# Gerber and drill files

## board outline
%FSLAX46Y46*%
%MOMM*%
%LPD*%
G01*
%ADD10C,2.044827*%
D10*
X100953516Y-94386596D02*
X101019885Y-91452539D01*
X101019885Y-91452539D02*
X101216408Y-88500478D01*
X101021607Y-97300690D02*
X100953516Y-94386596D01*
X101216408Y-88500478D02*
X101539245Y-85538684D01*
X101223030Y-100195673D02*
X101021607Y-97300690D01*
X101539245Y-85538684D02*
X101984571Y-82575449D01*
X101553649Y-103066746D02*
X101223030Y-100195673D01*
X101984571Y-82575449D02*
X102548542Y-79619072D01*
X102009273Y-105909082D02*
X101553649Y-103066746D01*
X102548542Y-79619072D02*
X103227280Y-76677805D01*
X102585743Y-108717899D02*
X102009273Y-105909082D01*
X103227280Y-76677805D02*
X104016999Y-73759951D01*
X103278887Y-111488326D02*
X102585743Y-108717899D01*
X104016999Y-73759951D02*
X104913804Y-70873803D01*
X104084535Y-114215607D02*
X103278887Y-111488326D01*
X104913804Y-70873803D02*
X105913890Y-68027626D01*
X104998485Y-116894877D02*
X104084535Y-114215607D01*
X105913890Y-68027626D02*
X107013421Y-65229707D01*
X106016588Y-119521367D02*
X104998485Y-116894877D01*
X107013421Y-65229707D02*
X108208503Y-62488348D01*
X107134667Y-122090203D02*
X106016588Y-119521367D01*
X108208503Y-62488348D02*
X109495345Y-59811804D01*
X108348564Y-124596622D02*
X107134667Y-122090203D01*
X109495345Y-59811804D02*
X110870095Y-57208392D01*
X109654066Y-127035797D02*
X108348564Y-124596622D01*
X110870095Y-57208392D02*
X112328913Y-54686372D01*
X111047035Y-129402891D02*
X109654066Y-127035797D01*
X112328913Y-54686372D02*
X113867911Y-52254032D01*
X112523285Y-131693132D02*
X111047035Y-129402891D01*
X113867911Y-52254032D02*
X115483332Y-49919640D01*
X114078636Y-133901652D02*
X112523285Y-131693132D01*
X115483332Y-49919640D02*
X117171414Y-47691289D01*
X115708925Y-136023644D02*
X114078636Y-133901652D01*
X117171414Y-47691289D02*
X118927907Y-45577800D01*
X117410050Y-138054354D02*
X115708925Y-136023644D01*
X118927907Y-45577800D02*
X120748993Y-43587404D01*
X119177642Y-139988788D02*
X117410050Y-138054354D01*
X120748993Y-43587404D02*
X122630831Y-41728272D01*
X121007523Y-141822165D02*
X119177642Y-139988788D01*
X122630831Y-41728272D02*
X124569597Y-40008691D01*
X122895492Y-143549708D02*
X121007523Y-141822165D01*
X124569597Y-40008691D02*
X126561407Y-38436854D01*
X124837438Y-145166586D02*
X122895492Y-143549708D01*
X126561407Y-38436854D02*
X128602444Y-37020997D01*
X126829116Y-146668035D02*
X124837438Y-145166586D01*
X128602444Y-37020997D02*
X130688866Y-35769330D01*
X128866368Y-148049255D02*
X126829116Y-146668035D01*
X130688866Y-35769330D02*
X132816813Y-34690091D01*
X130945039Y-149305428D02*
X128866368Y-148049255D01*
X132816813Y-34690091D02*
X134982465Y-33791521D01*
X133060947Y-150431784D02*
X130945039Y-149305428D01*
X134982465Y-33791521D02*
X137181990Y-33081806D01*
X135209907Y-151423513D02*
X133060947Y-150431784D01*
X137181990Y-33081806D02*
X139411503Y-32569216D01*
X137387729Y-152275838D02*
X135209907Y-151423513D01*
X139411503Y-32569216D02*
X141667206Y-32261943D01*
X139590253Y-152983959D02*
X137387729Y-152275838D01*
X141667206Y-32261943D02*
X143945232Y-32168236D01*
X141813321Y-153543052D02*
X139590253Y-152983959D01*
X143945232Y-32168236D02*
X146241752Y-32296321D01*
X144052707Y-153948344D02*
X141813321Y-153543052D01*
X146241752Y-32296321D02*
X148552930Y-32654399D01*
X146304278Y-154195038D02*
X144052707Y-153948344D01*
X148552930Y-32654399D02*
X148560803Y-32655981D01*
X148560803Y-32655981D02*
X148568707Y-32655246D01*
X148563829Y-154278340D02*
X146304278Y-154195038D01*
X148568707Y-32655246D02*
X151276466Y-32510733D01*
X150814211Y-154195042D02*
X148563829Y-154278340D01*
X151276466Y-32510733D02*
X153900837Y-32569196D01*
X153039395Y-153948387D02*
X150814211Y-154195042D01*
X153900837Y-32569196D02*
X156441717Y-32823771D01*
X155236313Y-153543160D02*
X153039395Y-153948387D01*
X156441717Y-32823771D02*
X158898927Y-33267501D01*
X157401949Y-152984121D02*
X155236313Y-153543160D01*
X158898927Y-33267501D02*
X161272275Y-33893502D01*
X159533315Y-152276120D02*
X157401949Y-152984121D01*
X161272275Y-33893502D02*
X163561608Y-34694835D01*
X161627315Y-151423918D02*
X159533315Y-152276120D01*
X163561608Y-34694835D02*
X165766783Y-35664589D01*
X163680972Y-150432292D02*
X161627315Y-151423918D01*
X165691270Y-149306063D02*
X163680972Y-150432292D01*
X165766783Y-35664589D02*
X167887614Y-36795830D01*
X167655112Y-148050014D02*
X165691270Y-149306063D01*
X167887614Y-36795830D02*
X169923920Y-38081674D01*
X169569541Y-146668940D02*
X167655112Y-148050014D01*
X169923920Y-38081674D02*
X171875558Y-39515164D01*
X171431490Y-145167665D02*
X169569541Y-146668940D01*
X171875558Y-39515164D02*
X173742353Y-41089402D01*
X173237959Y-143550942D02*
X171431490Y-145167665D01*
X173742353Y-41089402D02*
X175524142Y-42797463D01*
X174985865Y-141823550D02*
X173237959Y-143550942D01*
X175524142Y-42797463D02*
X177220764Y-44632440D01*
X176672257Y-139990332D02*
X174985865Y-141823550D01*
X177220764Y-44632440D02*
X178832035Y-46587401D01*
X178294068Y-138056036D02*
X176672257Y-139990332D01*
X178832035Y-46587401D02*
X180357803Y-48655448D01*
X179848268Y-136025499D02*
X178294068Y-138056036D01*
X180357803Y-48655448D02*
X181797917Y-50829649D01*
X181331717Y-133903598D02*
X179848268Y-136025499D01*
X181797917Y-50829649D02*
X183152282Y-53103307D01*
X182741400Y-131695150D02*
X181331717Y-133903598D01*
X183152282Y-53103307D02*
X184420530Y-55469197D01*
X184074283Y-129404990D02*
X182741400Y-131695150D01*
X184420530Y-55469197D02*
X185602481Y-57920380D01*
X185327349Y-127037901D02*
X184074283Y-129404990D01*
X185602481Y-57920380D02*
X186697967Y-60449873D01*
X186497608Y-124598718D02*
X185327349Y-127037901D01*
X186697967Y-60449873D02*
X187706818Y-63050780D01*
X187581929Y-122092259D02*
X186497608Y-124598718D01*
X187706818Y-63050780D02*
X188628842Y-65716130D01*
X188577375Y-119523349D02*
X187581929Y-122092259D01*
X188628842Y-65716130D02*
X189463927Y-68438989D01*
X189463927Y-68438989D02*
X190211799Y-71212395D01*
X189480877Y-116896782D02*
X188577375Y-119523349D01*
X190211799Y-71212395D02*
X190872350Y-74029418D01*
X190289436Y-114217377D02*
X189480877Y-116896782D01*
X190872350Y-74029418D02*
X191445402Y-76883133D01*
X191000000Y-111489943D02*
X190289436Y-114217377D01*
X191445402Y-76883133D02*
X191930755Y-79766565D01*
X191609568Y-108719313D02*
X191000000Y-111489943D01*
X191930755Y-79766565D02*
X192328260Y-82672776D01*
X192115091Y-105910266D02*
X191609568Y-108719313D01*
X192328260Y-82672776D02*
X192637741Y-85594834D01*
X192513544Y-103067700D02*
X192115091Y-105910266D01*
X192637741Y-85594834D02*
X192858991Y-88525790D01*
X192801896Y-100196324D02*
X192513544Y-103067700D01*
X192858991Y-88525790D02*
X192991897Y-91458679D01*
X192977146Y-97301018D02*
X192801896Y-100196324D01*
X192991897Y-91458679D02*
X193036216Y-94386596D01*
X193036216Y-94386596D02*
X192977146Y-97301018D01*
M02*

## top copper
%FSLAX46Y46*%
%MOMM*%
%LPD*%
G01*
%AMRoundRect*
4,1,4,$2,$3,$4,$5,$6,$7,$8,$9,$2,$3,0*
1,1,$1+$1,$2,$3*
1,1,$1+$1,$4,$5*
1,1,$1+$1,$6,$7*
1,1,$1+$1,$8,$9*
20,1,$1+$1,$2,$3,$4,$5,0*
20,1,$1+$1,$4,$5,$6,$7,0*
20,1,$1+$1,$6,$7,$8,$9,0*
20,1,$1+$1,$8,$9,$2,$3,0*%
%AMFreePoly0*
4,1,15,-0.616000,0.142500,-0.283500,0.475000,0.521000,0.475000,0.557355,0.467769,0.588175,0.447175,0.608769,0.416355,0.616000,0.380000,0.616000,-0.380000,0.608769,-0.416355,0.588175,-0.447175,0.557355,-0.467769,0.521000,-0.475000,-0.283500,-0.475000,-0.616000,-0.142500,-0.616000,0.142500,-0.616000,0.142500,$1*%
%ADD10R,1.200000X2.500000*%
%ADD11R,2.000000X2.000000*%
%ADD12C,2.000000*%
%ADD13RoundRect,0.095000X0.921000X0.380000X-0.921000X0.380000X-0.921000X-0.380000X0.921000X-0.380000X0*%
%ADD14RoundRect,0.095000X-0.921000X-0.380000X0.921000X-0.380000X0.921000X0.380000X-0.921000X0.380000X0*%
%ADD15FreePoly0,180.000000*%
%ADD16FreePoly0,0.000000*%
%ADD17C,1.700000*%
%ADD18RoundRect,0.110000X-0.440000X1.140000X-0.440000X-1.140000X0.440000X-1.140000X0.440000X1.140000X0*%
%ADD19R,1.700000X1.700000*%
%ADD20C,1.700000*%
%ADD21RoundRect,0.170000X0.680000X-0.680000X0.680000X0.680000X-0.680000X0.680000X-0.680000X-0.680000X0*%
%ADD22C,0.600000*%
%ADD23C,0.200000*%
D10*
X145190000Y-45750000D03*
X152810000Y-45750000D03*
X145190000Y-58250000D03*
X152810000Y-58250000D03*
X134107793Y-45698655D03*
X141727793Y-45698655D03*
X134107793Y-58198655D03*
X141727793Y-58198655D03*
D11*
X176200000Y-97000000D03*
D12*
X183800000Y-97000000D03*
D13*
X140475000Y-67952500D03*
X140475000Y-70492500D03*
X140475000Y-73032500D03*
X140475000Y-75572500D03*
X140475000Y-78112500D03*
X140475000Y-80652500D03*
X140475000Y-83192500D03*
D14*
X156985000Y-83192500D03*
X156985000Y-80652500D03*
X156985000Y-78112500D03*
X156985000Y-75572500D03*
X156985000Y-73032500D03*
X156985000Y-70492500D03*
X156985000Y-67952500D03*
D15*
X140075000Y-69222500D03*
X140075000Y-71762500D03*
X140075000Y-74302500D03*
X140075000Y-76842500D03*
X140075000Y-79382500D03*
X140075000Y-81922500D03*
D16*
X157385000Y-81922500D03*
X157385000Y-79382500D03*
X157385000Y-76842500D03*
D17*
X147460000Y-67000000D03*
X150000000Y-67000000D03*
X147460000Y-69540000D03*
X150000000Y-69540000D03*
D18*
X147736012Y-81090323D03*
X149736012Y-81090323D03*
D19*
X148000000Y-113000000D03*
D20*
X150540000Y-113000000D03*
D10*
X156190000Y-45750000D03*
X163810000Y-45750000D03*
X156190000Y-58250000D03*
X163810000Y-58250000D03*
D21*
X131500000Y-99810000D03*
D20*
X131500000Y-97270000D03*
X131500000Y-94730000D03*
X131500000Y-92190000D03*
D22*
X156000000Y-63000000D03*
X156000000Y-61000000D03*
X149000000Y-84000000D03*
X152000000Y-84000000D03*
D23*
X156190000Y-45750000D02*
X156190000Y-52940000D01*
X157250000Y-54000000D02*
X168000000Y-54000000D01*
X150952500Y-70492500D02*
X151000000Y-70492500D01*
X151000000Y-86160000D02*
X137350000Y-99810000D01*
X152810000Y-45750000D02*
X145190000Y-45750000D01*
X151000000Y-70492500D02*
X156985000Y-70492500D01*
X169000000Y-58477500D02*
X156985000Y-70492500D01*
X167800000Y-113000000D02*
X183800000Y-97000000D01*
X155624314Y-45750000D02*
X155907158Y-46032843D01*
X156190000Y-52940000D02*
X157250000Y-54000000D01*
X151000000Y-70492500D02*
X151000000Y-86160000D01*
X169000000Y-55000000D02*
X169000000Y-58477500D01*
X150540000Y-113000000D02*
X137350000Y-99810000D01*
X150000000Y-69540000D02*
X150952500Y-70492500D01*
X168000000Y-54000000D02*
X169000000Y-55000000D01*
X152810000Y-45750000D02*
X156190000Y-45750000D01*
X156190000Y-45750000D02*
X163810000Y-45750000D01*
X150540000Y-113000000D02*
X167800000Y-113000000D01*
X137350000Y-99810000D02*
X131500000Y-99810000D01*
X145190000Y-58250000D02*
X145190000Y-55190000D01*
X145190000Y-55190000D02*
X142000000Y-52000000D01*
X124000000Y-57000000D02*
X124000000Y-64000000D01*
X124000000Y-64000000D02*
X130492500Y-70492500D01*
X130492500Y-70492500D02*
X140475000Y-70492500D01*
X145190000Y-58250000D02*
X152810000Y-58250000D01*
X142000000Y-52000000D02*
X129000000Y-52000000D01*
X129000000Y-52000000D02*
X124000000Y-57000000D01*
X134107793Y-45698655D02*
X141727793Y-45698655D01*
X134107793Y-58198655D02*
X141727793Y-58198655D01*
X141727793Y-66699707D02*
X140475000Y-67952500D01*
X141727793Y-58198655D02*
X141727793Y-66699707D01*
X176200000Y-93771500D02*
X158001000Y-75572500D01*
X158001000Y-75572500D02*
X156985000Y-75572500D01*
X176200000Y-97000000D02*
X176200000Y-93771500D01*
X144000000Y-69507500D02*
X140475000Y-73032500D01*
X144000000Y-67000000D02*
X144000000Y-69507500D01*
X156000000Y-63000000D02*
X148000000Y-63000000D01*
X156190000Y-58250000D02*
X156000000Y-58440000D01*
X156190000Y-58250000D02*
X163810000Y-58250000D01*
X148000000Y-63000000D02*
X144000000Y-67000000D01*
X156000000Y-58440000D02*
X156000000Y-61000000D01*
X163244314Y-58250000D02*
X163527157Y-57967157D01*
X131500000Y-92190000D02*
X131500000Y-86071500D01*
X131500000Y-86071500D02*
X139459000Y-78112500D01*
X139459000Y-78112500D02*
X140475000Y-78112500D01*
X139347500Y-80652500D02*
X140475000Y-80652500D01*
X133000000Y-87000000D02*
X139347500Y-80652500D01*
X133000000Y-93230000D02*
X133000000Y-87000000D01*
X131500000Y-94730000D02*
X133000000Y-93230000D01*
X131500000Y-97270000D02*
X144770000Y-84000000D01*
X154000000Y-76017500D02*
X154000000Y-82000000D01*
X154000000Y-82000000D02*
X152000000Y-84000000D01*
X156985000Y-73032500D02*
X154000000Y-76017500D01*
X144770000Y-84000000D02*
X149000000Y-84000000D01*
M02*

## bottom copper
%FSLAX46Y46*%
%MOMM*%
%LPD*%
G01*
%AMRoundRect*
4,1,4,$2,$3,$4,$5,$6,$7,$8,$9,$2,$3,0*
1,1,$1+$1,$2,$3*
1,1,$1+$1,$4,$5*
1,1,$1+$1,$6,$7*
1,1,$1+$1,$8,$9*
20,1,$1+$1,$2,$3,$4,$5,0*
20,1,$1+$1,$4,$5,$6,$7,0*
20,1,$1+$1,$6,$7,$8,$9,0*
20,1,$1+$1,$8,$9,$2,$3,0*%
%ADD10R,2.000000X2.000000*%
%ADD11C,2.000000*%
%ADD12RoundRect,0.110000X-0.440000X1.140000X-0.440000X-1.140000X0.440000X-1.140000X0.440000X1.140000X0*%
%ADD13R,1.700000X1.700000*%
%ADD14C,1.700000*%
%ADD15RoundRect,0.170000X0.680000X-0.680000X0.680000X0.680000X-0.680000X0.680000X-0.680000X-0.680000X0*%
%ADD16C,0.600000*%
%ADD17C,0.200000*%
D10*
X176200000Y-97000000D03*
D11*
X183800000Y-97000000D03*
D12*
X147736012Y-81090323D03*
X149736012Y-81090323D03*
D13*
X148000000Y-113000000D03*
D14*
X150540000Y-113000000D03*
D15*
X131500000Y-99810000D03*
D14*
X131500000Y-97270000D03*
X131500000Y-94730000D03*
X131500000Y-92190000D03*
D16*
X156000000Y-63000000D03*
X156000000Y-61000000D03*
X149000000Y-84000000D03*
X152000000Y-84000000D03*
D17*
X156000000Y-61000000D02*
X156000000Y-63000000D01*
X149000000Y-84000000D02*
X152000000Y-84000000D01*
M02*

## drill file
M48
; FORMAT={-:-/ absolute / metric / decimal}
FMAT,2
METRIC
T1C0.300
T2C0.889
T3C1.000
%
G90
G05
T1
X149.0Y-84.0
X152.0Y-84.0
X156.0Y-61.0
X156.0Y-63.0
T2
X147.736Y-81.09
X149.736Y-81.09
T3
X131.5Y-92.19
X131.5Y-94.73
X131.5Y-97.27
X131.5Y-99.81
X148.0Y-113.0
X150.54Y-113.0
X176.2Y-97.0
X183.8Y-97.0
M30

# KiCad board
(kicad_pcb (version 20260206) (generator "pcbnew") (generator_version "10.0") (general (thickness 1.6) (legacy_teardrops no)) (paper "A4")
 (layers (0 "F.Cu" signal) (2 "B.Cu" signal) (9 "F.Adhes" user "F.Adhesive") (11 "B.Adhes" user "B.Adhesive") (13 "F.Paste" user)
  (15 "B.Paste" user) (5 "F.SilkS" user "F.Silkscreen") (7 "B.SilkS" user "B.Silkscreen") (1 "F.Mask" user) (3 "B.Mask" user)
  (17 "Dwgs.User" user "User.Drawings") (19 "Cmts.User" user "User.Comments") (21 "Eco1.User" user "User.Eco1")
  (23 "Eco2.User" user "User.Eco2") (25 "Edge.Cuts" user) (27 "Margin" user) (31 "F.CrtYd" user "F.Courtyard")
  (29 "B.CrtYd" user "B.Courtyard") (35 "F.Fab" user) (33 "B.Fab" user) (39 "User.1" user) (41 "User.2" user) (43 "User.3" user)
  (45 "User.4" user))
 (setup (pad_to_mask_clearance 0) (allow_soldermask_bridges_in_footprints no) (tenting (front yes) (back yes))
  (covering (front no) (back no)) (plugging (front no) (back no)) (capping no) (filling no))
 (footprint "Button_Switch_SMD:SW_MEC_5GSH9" (layer "F.Cu") (at 149 52)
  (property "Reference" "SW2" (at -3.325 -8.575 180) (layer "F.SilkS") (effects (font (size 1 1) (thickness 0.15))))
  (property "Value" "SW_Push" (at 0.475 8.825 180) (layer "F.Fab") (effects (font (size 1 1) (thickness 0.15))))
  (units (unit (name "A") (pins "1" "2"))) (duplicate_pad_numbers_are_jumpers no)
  (pad "1" smd rect (at -3.81 -6.25 90) (size 2.5 1.2) (layers "F.Cu" "F.Mask" "F.Paste") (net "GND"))
  (pad "1" smd rect (at 3.81 -6.25 90) (size 2.5 1.2) (layers "F.Cu" "F.Mask" "B.SilkS" "F.Paste") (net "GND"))
  (pad "2" smd rect (at -3.81 6.25 90) (size 2.5 1.2) (layers "F.Cu" "F.Mask" "F.Paste") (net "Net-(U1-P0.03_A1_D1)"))
  (pad "2" smd rect (at 3.81 6.25 90) (size 2.5 1.2) (layers "F.Cu" "F.Mask" "F.Paste") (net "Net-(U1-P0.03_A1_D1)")))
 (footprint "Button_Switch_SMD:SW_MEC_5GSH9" (layer "F.Cu") (at 137.917793 51.948655)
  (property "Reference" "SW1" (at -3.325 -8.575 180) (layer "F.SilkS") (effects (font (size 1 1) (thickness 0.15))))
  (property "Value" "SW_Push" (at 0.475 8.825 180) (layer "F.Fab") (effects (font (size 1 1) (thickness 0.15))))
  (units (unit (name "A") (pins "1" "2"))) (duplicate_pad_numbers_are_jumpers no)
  (pad "1" smd rect (at -3.81 -6.25 90) (size 2.5 1.2) (layers "F.Cu" "F.Mask" "F.Paste") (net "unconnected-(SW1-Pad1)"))
  (pad "1" smd rect (at 3.81 -6.25 90) (size 2.5 1.2) (layers "F.Cu" "F.Mask" "B.SilkS" "F.Paste") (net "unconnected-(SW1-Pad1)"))
  (pad "2" smd rect (at -3.81 6.25 90) (size 2.5 1.2) (layers "F.Cu" "F.Mask" "F.Paste") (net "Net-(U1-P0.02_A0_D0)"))
  (pad "2" smd rect (at 3.81 6.25 90) (size 2.5 1.2) (layers "F.Cu" "F.Mask" "F.Paste") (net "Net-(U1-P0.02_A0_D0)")))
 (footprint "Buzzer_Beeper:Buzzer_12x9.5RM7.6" (layer "F.Cu") (at 176.2 97)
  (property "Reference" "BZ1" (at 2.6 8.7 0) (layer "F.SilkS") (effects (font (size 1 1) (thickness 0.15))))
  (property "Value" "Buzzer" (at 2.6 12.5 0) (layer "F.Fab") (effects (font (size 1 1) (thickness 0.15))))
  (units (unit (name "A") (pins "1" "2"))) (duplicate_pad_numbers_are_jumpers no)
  (pad "1" thru_hole rect (at 0 0) (size 2 2) (drill 1) (layers "*.Cu" "*.Mask") (remove_unused_layers no) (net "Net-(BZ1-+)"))
  (pad "2" thru_hole circle (at 7.6 0) (size 2 2) (drill 1) (layers "*.Cu" "*.Mask") (remove_unused_layers no) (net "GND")))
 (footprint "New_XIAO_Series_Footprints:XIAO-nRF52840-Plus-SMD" (layer "F.Cu") (at 148.73 75.5725 90)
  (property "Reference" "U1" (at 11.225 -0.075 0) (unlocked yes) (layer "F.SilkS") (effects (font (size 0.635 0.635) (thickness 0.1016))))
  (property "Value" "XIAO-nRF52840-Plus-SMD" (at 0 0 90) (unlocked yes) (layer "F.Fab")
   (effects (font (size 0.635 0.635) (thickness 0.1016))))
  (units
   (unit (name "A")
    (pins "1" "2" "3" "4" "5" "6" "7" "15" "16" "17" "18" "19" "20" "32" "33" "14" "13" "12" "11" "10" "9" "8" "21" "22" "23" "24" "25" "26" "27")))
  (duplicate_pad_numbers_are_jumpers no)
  (pad "1" smd roundrect (at 7.62 -8.255 180) (size 2.032 0.95) (layers "F.Cu" "F.Mask" "F.Paste") (roundrect_rratio 0.1)
   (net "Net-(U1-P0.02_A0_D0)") (thermal_bridge_angle 45))
  (pad "2" smd roundrect (at 5.08 -8.255 180) (size 2.032 0.95) (layers "F.Cu" "F.Mask" "F.Paste") (roundrect_rratio 0.1)
   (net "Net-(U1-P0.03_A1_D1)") (thermal_bridge_angle 45))
  (pad "3" smd roundrect (at 2.54 -8.255 180) (size 2.032 0.95) (layers "F.Cu" "F.Mask" "F.Paste") (roundrect_rratio 0.1)
   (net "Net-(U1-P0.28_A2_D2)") (thermal_bridge_angle 45))
  (pad "4" smd roundrect (at 0 -8.255 180) (size 2.032 0.95) (layers "F.Cu" "F.Mask" "F.Paste") (roundrect_rratio 0.1)
   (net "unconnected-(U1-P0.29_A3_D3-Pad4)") (thermal_bridge_angle 45))
  (pad "5" smd roundrect (at -2.54 -8.255 180) (size 2.032 0.95) (layers "F.Cu" "F.Mask" "F.Paste") (roundrect_rratio 0.1)
   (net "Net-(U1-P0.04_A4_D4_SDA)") (thermal_bridge_angle 45))
  (pad "6" smd roundrect (at -5.08 -8.255 180) (size 2.032 0.95) (layers "F.Cu" "F.Mask" "F.Paste") (roundrect_rratio 0.1)
   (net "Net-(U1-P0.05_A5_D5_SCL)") (thermal_bridge_angle 45))
  (pad "7" smd roundrect (at -7.62 -8.255 180) (size 2.032 0.95) (layers "F.Cu" "F.Mask" "F.Paste") (roundrect_rratio 0.1)
   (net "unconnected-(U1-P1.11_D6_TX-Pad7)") (thermal_bridge_angle 45))
  (pad "8" smd roundrect (at -7.62 8.255) (size 2.032 0.95) (layers "F.Cu" "F.Mask" "F.Paste") (roundrect_rratio 0.1)
   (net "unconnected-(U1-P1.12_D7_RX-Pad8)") (thermal_bridge_angle 45))
  (pad "9" smd roundrect (at -5.08 8.255) (size 2.032 0.95) (layers "F.Cu" "F.Mask" "F.Paste") (roundrect_rratio 0.1)
   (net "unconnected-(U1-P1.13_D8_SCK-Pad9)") (thermal_bridge_angle 45))
  (pad "10" smd roundrect (at -2.54 8.255) (size 2.032 0.95) (layers "F.Cu" "F.Mask" "F.Paste") (roundrect_rratio 0.1)
   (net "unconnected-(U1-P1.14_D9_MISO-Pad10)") (thermal_bridge_angle 45))
  (pad "11" smd roundrect (at 0 8.255) (size 2.032 0.95) (layers "F.Cu" "F.Mask" "F.Paste") (roundrect_rratio 0.1) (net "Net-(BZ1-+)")
   (thermal_bridge_angle 45))
  (pad "12" smd roundrect (at 2.54 8.255) (size 2.032 0.95) (layers "F.Cu" "F.Mask" "F.Paste") (roundrect_rratio 0.1) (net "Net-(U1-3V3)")
   (thermal_bridge_angle 45))
  (pad "13" smd roundrect (at 5.08 8.255) (size 2.032 0.95) (layers "F.Cu" "F.Mask" "F.Paste") (roundrect_rratio 0.1) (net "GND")
   (thermal_bridge_angle 45))
  (pad "14" smd roundrect (at 7.62 8.255) (size 2.032 0.95) (layers "F.Cu" "F.Mask" "F.Paste") (roundrect_rratio 0.1)
   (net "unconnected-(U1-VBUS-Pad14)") (thermal_bridge_angle 45))
  (pad "15" smd roundrect (at 6.35 -8.655 180) (size 1.232 0.95) (layers "F.Cu" "F.Mask" "F.Paste") (roundrect_rratio 0.1)
   (chamfer_ratio 0.35) (chamfer top_left bottom_left) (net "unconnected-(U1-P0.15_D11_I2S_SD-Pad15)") (thermal_bridge_angle 45))
  (pad "16" smd roundrect (at 3.81 -8.655 180) (size 1.232 0.95) (layers "F.Cu" "F.Mask" "F.Paste") (roundrect_rratio 0.1)
   (chamfer_ratio 0.35) (chamfer top_left bottom_left) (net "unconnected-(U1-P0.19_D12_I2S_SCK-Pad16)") (thermal_bridge_angle 45))
  (pad "17" smd roundrect (at 1.27 -8.655 180) (size 1.232 0.95) (layers "F.Cu" "F.Mask" "F.Paste") (roundrect_rratio 0.1)
   (chamfer_ratio 0.35) (chamfer top_left bottom_left) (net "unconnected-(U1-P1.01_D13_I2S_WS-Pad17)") (thermal_bridge_angle 45))
  (pad "18" smd roundrect (at -1.27 -8.655 180) (size 1.232 0.95) (layers "F.Cu" "F.Mask" "F.Paste") (roundrect_rratio 0.1)
   (chamfer_ratio 0.35) (chamfer top_left bottom_left) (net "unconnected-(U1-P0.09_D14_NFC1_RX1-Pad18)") (thermal_bridge_angle 45))
  (pad "19" smd roundrect (at -3.81 -8.655 180) (size 1.232 0.95) (layers "F.Cu" "F.Mask" "F.Paste") (roundrect_rratio 0.1)
   (chamfer_ratio 0.35) (chamfer top_left bottom_left) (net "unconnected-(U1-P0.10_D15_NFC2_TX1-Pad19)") (thermal_bridge_angle 45))
  (pad "20" smd roundrect (at -6.35 -8.655 180) (size 1.232 0.95) (layers "F.Cu" "F.Mask" "F.Paste") (roundrect_rratio 0.1)
   (chamfer_ratio 0.35) (chamfer top_left bottom_left) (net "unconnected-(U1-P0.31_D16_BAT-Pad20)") (thermal_bridge_angle 45))
  (pad "21" smd roundrect (at -6.35 8.655) (size 1.232 0.95) (layers "F.Cu" "F.Mask" "F.Paste") (roundrect_rratio 0.1) (chamfer_ratio 0.35)
   (chamfer top_left bottom_left) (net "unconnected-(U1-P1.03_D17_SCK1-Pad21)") (thermal_bridge_angle 45))
  (pad "22" smd roundrect (at -3.81 8.655) (size 1.232 0.95) (layers "F.Cu" "F.Mask" "F.Paste") (roundrect_rratio 0.1) (chamfer_ratio 0.35)
   (chamfer top_left bottom_left) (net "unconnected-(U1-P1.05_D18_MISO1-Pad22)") (thermal_bridge_angle 45))
  (pad "23" smd roundrect (at -1.27 8.655) (size 1.232 0.95) (layers "F.Cu" "F.Mask" "F.Paste") (roundrect_rratio 0.1) (chamfer_ratio 0.35)
   (chamfer top_left bottom_left) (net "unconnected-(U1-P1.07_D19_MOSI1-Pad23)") (thermal_bridge_angle 45))
  (pad "24" smd circle (at 8.5725 -1.27) (size 1.7 1.7) (layers "F.Cu" "F.Mask" "F.Paste") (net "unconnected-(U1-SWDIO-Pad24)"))
  (pad "25" smd circle (at 8.5725 1.27) (size 1.7 1.7) (layers "F.Cu" "F.Mask" "F.Paste") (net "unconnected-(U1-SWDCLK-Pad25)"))
  (pad "26" smd circle (at 6.0325 -1.27) (size 1.7 1.7) (layers "F.Cu" "F.Mask" "F.Paste") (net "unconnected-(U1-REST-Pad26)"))
  (pad "27" smd circle (at 6.0325 1.27) (size 1.7 1.7) (layers "F.Cu" "F.Mask" "F.Paste") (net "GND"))
  (pad "28" thru_hole roundrect (at -5.517823 -0.993988 270) (size 2.5 1.1) (drill 0.889) (layers "*.Cu" "*.Mask") (remove_unused_layers no)
   (roundrect_rratio 0.1) (thermal_bridge_angle 45))
  (pad "29" thru_hole roundrect (at -5.517823 1.006012 270) (size 2.5 1.1) (drill 0.889) (layers "*.Cu" "*.Mask") (remove_unused_layers no)
   (roundrect_rratio 0.1) (thermal_bridge_angle 45)))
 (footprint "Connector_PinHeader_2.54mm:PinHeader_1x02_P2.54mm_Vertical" (layer "F.Cu") (at 148 113 90)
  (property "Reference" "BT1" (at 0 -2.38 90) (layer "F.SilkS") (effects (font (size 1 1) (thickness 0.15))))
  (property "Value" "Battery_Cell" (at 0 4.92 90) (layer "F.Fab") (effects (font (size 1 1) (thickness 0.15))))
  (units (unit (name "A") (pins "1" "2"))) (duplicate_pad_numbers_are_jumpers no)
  (pad "1" thru_hole rect (at 0 0 90) (size 1.7 1.7) (drill 1) (layers "*.Cu" "*.Mask") (remove_unused_layers no) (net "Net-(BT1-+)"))
  (pad "2" thru_hole circle (at 0 2.54 90) (size 1.7 1.7) (drill 1) (layers "*.Cu" "*.Mask") (remove_unused_layers no) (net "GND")))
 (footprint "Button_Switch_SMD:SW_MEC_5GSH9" (layer "F.Cu") (at 160 52)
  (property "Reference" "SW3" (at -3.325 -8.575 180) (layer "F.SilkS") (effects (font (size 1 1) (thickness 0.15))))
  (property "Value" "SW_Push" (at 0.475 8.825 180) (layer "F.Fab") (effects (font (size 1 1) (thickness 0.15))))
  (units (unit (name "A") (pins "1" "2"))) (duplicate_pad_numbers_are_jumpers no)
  (pad "1" smd rect (at -3.81 -6.25 90) (size 2.5 1.2) (layers "F.Cu" "F.Mask" "F.Paste") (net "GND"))
  (pad "1" smd rect (at 3.81 -6.25 90) (size 2.5 1.2) (layers "F.Cu" "F.Mask" "B.SilkS" "F.Paste") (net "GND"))
  (pad "2" smd rect (at -3.81 6.25 90) (size 2.5 1.2) (layers "F.Cu" "F.Mask" "F.Paste") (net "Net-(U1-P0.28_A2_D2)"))
  (pad "2" smd rect (at 3.81 6.25 90) (size 2.5 1.2) (layers "F.Cu" "F.Mask" "F.Paste") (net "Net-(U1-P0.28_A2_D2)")))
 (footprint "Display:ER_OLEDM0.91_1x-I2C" (layer "F.Cu") (at 131.5 99.81 90)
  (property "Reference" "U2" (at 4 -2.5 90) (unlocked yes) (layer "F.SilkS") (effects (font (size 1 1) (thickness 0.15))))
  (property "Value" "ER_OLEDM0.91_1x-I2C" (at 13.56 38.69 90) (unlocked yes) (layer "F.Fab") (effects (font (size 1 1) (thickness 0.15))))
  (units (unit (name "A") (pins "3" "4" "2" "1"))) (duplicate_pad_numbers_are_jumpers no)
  (pad "1" thru_hole roundrect (at 0 0 90) (size 1.7 1.7) (drill 1) (layers "*.Cu" "*.Mask") (remove_unused_layers no)
   (roundrect_rratio 0.1) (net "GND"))
  (pad "2" thru_hole circle (at 2.54 0 90) (size 1.7 1.7) (drill 1) (layers "*.Cu" "*.Mask") (remove_unused_layers no) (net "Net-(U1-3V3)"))
  (pad "3" thru_hole circle (at 5.08 0 90) (size 1.7 1.7) (drill 1) (layers "*.Cu" "*.Mask") (remove_unused_layers no)
   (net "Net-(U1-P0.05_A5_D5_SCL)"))
  (pad "4" thru_hole circle (at 7.62 0 90) (size 1.7 1.7) (drill 1) (layers "*.Cu" "*.Mask") (remove_unused_layers no)
   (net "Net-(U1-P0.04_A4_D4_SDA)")))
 (gr_line (start 100.953516 94.386596) (end 101.019885 91.452539) (stroke (width 2.044827) (type default)) (layer "Edge.Cuts"))
 (gr_line (start 101.019885 91.452539) (end 101.216408 88.500478) (stroke (width 2.044827) (type default)) (layer "Edge.Cuts"))
 (gr_line (start 101.021607 97.30069) (end 100.953516 94.386596) (stroke (width 2.044827) (type default)) (layer "Edge.Cuts"))
 (gr_line (start 101.216408 88.500478) (end 101.539245 85.538684) (stroke (width 2.044827) (type default)) (layer "Edge.Cuts"))
 (gr_line (start 101.22303 100.195673) (end 101.021607 97.30069) (stroke (width 2.044827) (type default)) (layer "Edge.Cuts"))
 (gr_line (start 101.539245 85.538684) (end 101.984571 82.575449) (stroke (width 2.044827) (type default)) (layer "Edge.Cuts"))
 (gr_line (start 101.553649 103.066746) (end 101.22303 100.195673) (stroke (width 2.044827) (type default)) (layer "Edge.Cuts"))
 (gr_line (start 101.984571 82.575449) (end 102.548542 79.619072) (stroke (width 2.044827) (type default)) (layer "Edge.Cuts"))
 (gr_line (start 102.009273 105.909082) (end 101.553649 103.066746) (stroke (width 2.044827) (type default)) (layer "Edge.Cuts"))
 (gr_line (start 102.548542 79.619072) (end 103.22728 76.677805) (stroke (width 2.044827) (type default)) (layer "Edge.Cuts"))
 (gr_line (start 102.585743 108.717899) (end 102.009273 105.909082) (stroke (width 2.044827) (type default)) (layer "Edge.Cuts"))
 (gr_line (start 103.22728 76.677805) (end 104.016999 73.759951) (stroke (width 2.044827) (type default)) (layer "Edge.Cuts"))
 (gr_line (start 103.278887 111.488326) (end 102.585743 108.717899) (stroke (width 2.044827) (type default)) (layer "Edge.Cuts"))
 (gr_line (start 104.016999 73.759951) (end 104.913804 70.873803) (stroke (width 2.044827) (type default)) (layer "Edge.Cuts"))
 (gr_line (start 104.084535 114.215607) (end 103.278887 111.488326) (stroke (width 2.044827) (type default)) (layer "Edge.Cuts"))
 (gr_line (start 104.913804 70.873803) (end 105.91389 68.027626) (stroke (width 2.044827) (type default)) (layer "Edge.Cuts"))
 (gr_line (start 104.998485 116.894877) (end 104.084535 114.215607) (stroke (width 2.044827) (type default)) (layer "Edge.Cuts"))
 (gr_line (start 105.91389 68.027626) (end 107.013421 65.229707) (stroke (width 2.044827) (type default)) (layer "Edge.Cuts"))
 (gr_line (start 106.016588 119.521367) (end 104.998485 116.894877) (stroke (width 2.044827) (type default)) (layer "Edge.Cuts"))
 (gr_line (start 107.013421 65.229707) (end 108.208503 62.488348) (stroke (width 2.044827) (type default)) (layer "Edge.Cuts"))
 (gr_line (start 107.134667 122.090203) (end 106.016588 119.521367) (stroke (width 2.044827) (type default)) (layer "Edge.Cuts"))
 (gr_line (start 108.208503 62.488348) (end 109.495345 59.811804) (stroke (width 2.044827) (type default)) (layer "Edge.Cuts"))
 (gr_line (start 108.348564 124.596622) (end 107.134667 122.090203) (stroke (width 2.044827) (type default)) (layer "Edge.Cuts"))
 (gr_line (start 109.495345 59.811804) (end 110.870095 57.208392) (stroke (width 2.044827) (type default)) (layer "Edge.Cuts"))
 (gr_line (start 109.654066 127.035797) (end 108.348564 124.596622) (stroke (width 2.044827) (type default)) (layer "Edge.Cuts"))
 (gr_line (start 110.870095 57.208392) (end 112.328913 54.686372) (stroke (width 2.044827) (type default)) (layer "Edge.Cuts"))
 (gr_line (start 111.047035 129.402891) (end 109.654066 127.035797) (stroke (width 2.044827) (type default)) (layer "Edge.Cuts"))
 (gr_line (start 112.328913 54.686372) (end 113.867911 52.254032) (stroke (width 2.044827) (type default)) (layer "Edge.Cuts"))
 (gr_line (start 112.523285 131.693132) (end 111.047035 129.402891) (stroke (width 2.044827) (type default)) (layer "Edge.Cuts"))
 (gr_line (start 113.867911 52.254032) (end 115.483332 49.91964) (stroke (width 2.044827) (type default)) (layer "Edge.Cuts"))
 (gr_line (start 114.078636 133.901652) (end 112.523285 131.693132) (stroke (width 2.044827) (type default)) (layer "Edge.Cuts"))
 (gr_line (start 115.483332 49.91964) (end 117.171414 47.691289) (stroke (width 2.044827) (type default)) (layer "Edge.Cuts"))
 (gr_line (start 115.708925 136.023644) (end 114.078636 133.901652) (stroke (width 2.044827) (type default)) (layer "Edge.Cuts"))
 (gr_line (start 117.171414 47.691289) (end 118.927907 45.5778) (stroke (width 2.044827) (type default)) (layer "Edge.Cuts"))
 (gr_line (start 117.41005 138.054354) (end 115.708925 136.023644) (stroke (width 2.044827) (type default)) (layer "Edge.Cuts"))
 (gr_line (start 118.927907 45.5778) (end 120.748993 43.587404) (stroke (width 2.044827) (type default)) (layer "Edge.Cuts"))
 (gr_line (start 119.177642 139.988788) (end 117.41005 138.054354) (stroke (width 2.044827) (type default)) (layer "Edge.Cuts"))
 (gr_line (start 120.748993 43.587404) (end 122.630831 41.728272) (stroke (width 2.044827) (type default)) (layer "Edge.Cuts"))
 (gr_line (start 121.007523 141.822165) (end 119.177642 139.988788) (stroke (width 2.044827) (type default)) (layer "Edge.Cuts"))
 (gr_line (start 122.630831 41.728272) (end 124.569597 40.008691) (stroke (width 2.044827) (type default)) (layer "Edge.Cuts"))
 (gr_line (start 122.895492 143.549708) (end 121.007523 141.822165) (stroke (width 2.044827) (type default)) (layer "Edge.Cuts"))
 (gr_line (start 124.569597 40.008691) (end 126.561407 38.436854) (stroke (width 2.044827) (type default)) (layer "Edge.Cuts"))
 (gr_line (start 124.837438 145.166586) (end 122.895492 143.549708) (stroke (width 2.044827) (type default)) (layer "Edge.Cuts"))
 (gr_line (start 126.561407 38.436854) (end 128.602444 37.020997) (stroke (width 2.044827) (type default)) (layer "Edge.Cuts"))
 (gr_line (start 126.829116 146.668035) (end 124.837438 145.166586) (stroke (width 2.044827) (type default)) (layer "Edge.Cuts"))
 (gr_line (start 128.602444 37.020997) (end 130.688866 35.76933) (stroke (width 2.044827) (type default)) (layer "Edge.Cuts"))
 (gr_line (start 128.866368 148.049255) (end 126.829116 146.668035) (stroke (width 2.044827) (type default)) (layer "Edge.Cuts"))
 (gr_line (start 130.688866 35.76933) (end 132.816813 34.690091) (stroke (width 2.044827) (type default)) (layer "Edge.Cuts"))
 (gr_line (start 130.945039 149.305428) (end 128.866368 148.049255) (stroke (width 2.044827) (type default)) (layer "Edge.Cuts"))
 (gr_line (start 132.816813 34.690091) (end 134.982465 33.791521) (stroke (width 2.044827) (type default)) (layer "Edge.Cuts"))
 (gr_line (start 133.060947 150.431784) (end 130.945039 149.305428) (stroke (width 2.044827) (type default)) (layer "Edge.Cuts"))
 (gr_line (start 134.982465 33.791521) (end 137.18199 33.081806) (stroke (width 2.044827) (type default)) (layer "Edge.Cuts"))
 (gr_line (start 135.209907 151.423513) (end 133.060947 150.431784) (stroke (width 2.044827) (type default)) (layer "Edge.Cuts"))
 (gr_line (start 137.18199 33.081806) (end 139.411503 32.569216) (stroke (width 2.044827) (type default)) (layer "Edge.Cuts"))
 (gr_line (start 137.387729 152.275838) (end 135.209907 151.423513) (stroke (width 2.044827) (type default)) (layer "Edge.Cuts"))
 (gr_line (start 139.411503 32.569216) (end 141.667206 32.261943) (stroke (width 2.044827) (type default)) (layer "Edge.Cuts"))
 (gr_line (start 139.590253 152.983959) (end 137.387729 152.275838) (stroke (width 2.044827) (type default)) (layer "Edge.Cuts"))
 (gr_line (start 141.667206 32.261943) (end 143.945232 32.168236) (stroke (width 2.044827) (type default)) (layer "Edge.Cuts"))
 (gr_line (start 141.813321 153.543052) (end 139.590253 152.983959) (stroke (width 2.044827) (type default)) (layer "Edge.Cuts"))
 (gr_line (start 143.945232 32.168236) (end 146.241752 32.296321) (stroke (width 2.044827) (type default)) (layer "Edge.Cuts"))
 (gr_line (start 144.052707 153.948344) (end 141.813321 153.543052) (stroke (width 2.044827) (type default)) (layer "Edge.Cuts"))
 (gr_line (start 146.241752 32.296321) (end 148.55293 32.654399) (stroke (width 2.044827) (type default)) (layer "Edge.Cuts"))
 (gr_line (start 146.304278 154.195038) (end 144.052707 153.948344) (stroke (width 2.044827) (type default)) (layer "Edge.Cuts"))
 (gr_line (start 148.55293 32.654399) (end 148.560803 32.655981) (stroke (width 2.044827) (type default)) (layer "Edge.Cuts"))
 (gr_line (start 148.560803 32.655981) (end 148.568707 32.655246) (stroke (width 2.044827) (type default)) (layer "Edge.Cuts"))
 (gr_line (start 148.563829 154.27834) (end 146.304278 154.195038) (stroke (width 2.044827) (type default)) (layer "Edge.Cuts"))
 (gr_line (start 148.568707 32.655246) (end 151.276466 32.510733) (stroke (width 2.044827) (type default)) (layer "Edge.Cuts"))
 (gr_line (start 150.814211 154.195042) (end 148.563829 154.27834) (stroke (width 2.044827) (type default)) (layer "Edge.Cuts"))
 (gr_line (start 151.276466 32.510733) (end 153.900837 32.569196) (stroke (width 2.044827) (type default)) (layer "Edge.Cuts"))
 (gr_line (start 153.039395 153.948387) (end 150.814211 154.195042) (stroke (width 2.044827) (type default)) (layer "Edge.Cuts"))
 (gr_line (start 153.900837 32.569196) (end 156.441717 32.823771) (stroke (width 2.044827) (type default)) (layer "Edge.Cuts"))
 (gr_line (start 155.236313 153.54316) (end 153.039395 153.948387) (stroke (width 2.044827) (type default)) (layer "Edge.Cuts"))
 (gr_line (start 156.441717 32.823771) (end 158.898927 33.267501) (stroke (width 2.044827) (type default)) (layer "Edge.Cuts"))
 (gr_line (start 157.401949 152.984121) (end 155.236313 153.54316) (stroke (width 2.044827) (type default)) (layer "Edge.Cuts"))
 (gr_line (start 158.898927 33.267501) (end 161.272275 33.893502) (stroke (width 2.044827) (type default)) (layer "Edge.Cuts"))
 (gr_line (start 159.533315 152.27612) (end 157.401949 152.984121) (stroke (width 2.044827) (type default)) (layer "Edge.Cuts"))
 (gr_line (start 161.272275 33.893502) (end 163.561608 34.694835) (stroke (width 2.044827) (type default)) (layer "Edge.Cuts"))
 (gr_line (start 161.627315 151.423918) (end 159.533315 152.27612) (stroke (width 2.044827) (type default)) (layer "Edge.Cuts"))
 (gr_line (start 163.561608 34.694835) (end 165.766783 35.664589) (stroke (width 2.044827) (type default)) (layer "Edge.Cuts"))
 (gr_line (start 163.680972 150.432292) (end 161.627315 151.423918) (stroke (width 2.044827) (type default)) (layer "Edge.Cuts"))
 (gr_line (start 165.69127 149.306063) (end 163.680972 150.432292) (stroke (width 2.044827) (type default)) (layer "Edge.Cuts"))
 (gr_line (start 165.766783 35.664589) (end 167.887614 36.79583) (stroke (width 2.044827) (type default)) (layer "Edge.Cuts"))
 (gr_line (start 167.655112 148.050014) (end 165.69127 149.306063) (stroke (width 2.044827) (type default)) (layer "Edge.Cuts"))
 (gr_line (start 167.887614 36.79583) (end 169.92392 38.081674) (stroke (width 2.044827) (type default)) (layer "Edge.Cuts"))
 (gr_line (start 169.569541 146.66894) (end 167.655112 148.050014) (stroke (width 2.044827) (type default)) (layer "Edge.Cuts"))
 (gr_line (start 169.92392 38.081674) (end 171.875558 39.515164) (stroke (width 2.044827) (type default)) (layer "Edge.Cuts"))
 (gr_line (start 171.43149 145.167665) (end 169.569541 146.66894) (stroke (width 2.044827) (type default)) (layer "Edge.Cuts"))
 (gr_line (start 171.875558 39.515164) (end 173.742353 41.089402) (stroke (width 2.044827) (type default)) (layer "Edge.Cuts"))
 (gr_line (start 173.237959 143.550942) (end 171.43149 145.167665) (stroke (width 2.044827) (type default)) (layer "Edge.Cuts"))
 (gr_line (start 173.742353 41.089402) (end 175.524142 42.797463) (stroke (width 2.044827) (type default)) (layer "Edge.Cuts"))
 (gr_line (start 174.985865 141.82355) (end 173.237959 143.550942) (stroke (width 2.044827) (type default)) (layer "Edge.Cuts"))
 (gr_line (start 175.524142 42.797463) (end 177.220764 44.63244) (stroke (width 2.044827) (type default)) (layer "Edge.Cuts"))
 (gr_line (start 176.672257 139.990332) (end 174.985865 141.82355) (stroke (width 2.044827) (type default)) (layer "Edge.Cuts"))
 (gr_line (start 177.220764 44.63244) (end 178.832035 46.587401) (stroke (width 2.044827) (type default)) (layer "Edge.Cuts"))
 (gr_line (start 178.294068 138.056036) (end 176.672257 139.990332) (stroke (width 2.044827) (type default)) (layer "Edge.Cuts"))
 (gr_line (start 178.832035 46.587401) (end 180.357803 48.655448) (stroke (width 2.044827) (type default)) (layer "Edge.Cuts"))
 (gr_line (start 179.848268 136.025499) (end 178.294068 138.056036) (stroke (width 2.044827) (type default)) (layer "Edge.Cuts"))
 (gr_line (start 180.357803 48.655448) (end 181.797917 50.829649) (stroke (width 2.044827) (type default)) (layer "Edge.Cuts"))
 (gr_line (start 181.331717 133.903598) (end 179.848268 136.025499) (stroke (width 2.044827) (type default)) (layer "Edge.Cuts"))
 (gr_line (start 181.797917 50.829649) (end 183.152282 53.103307) (stroke (width 2.044827) (type default)) (layer "Edge.Cuts"))
 (gr_line (start 182.7414 131.69515) (end 181.331717 133.903598) (stroke (width 2.044827) (type default)) (layer "Edge.Cuts"))
 (gr_line (start 183.152282 53.103307) (end 184.42053 55.469197) (stroke (width 2.044827) (type default)) (layer "Edge.Cuts"))
 (gr_line (start 184.074283 129.40499) (end 182.7414 131.69515) (stroke (width 2.044827) (type default)) (layer "Edge.Cuts"))
 (gr_line (start 184.42053 55.469197) (end 185.602481 57.92038) (stroke (width 2.044827) (type default)) (layer "Edge.Cuts"))
 (gr_line (start 185.327349 127.037901) (end 184.074283 129.40499) (stroke (width 2.044827) (type default)) (layer "Edge.Cuts"))
 (gr_line (start 185.602481 57.92038) (end 186.697967 60.449873) (stroke (width 2.044827) (type default)) (layer "Edge.Cuts"))
 (gr_line (start 186.497608 124.598718) (end 185.327349 127.037901) (stroke (width 2.044827) (type default)) (layer "Edge.Cuts"))
 (gr_line (start 186.697967 60.449873) (end 187.706818 63.05078) (stroke (width 2.044827) (type default)) (layer "Edge.Cuts"))
 (gr_line (start 187.581929 122.092259) (end 186.497608 124.598718) (stroke (width 2.044827) (type default)) (layer "Edge.Cuts"))
 (gr_line (start 187.706818 63.05078) (end 188.628842 65.71613) (stroke (width 2.044827) (type default)) (layer "Edge.Cuts"))
 (gr_line (start 188.577375 119.523349) (end 187.581929 122.092259) (stroke (width 2.044827) (type default)) (layer "Edge.Cuts"))
 (gr_line (start 188.628842 65.71613) (end 189.463927 68.438989) (stroke (width 2.044827) (type default)) (layer "Edge.Cuts"))
 (gr_line (start 189.463927 68.438989) (end 190.211799 71.212395) (stroke (width 2.044827) (type default)) (layer "Edge.Cuts"))
 (gr_line (start 189.480877 116.896782) (end 188.577375 119.523349) (stroke (width 2.044827) (type default)) (layer "Edge.Cuts"))
 (gr_line (start 190.211799 71.212395) (end 190.87235 74.029418) (stroke (width 2.044827) (type default)) (layer "Edge.Cuts"))
 (gr_line (start 190.289436 114.217377) (end 189.480877 116.896782) (stroke (width 2.044827) (type default)) (layer "Edge.Cuts"))
 (gr_line (start 190.87235 74.029418) (end 191.445402 76.883133) (stroke (width 2.044827) (type default)) (layer "Edge.Cuts"))
 (gr_line (start 191 111.489943) (end 190.289436 114.217377) (stroke (width 2.044827) (type default)) (layer "Edge.Cuts"))
 (gr_line (start 191.445402 76.883133) (end 191.930755 79.766565) (stroke (width 2.044827) (type default)) (layer "Edge.Cuts"))
 (gr_line (start 191.609568 108.719313) (end 191 111.489943) (stroke (width 2.044827) (type default)) (layer "Edge.Cuts"))
 (gr_line (start 191.930755 79.766565) (end 192.32826 82.672776) (stroke (width 2.044827) (type default)) (layer "Edge.Cuts"))
 (gr_line (start 192.115091 105.910266) (end 191.609568 108.719313) (stroke (width 2.044827) (type default)) (layer "Edge.Cuts"))
 (gr_line (start 192.32826 82.672776) (end 192.637741 85.594834) (stroke (width 2.044827) (type default)) (layer "Edge.Cuts"))
 (gr_line (start 192.513544 103.0677) (end 192.115091 105.910266) (stroke (width 2.044827) (type default)) (layer "Edge.Cuts"))
 (gr_line (start 192.637741 85.594834) (end 192.858991 88.52579) (stroke (width 2.044827) (type default)) (layer "Edge.Cuts"))
 (gr_line (start 192.801896 100.196324) (end 192.513544 103.0677) (stroke (width 2.044827) (type default)) (layer "Edge.Cuts"))
 (gr_line (start 192.858991 88.52579) (end 192.991897 91.458679) (stroke (width 2.044827) (type default)) (layer "Edge.Cuts"))
 (gr_line (start 192.977146 97.301018) (end 192.801896 100.196324) (stroke (width 2.044827) (type default)) (layer "Edge.Cuts"))
 (gr_line (start 192.991897 91.458679) (end 193.036216 94.386596) (stroke (width 2.044827) (type default)) (layer "Edge.Cuts"))
 (gr_line (start 193.036216 94.386596) (end 192.977146 97.301018) (stroke (width 2.044827) (type default)) (layer "Edge.Cuts"))
 (segment (start 156.19 45.75) (end 156.19 52.94) (width 0.2) (layer "F.Cu") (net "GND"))
 (segment (start 157.25 54) (end 168 54) (width 0.2) (layer "F.Cu") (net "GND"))
 (segment (start 150.9525 70.4925) (end 151 70.4925) (width 0.2) (layer "F.Cu") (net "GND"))
 (segment (start 151 86.16) (end 137.35 99.81) (width 0.2) (layer "F.Cu") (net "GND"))
 (segment (start 152.81 45.75) (end 145.19 45.75) (width 0.2) (layer "F.Cu") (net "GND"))
 (segment (start 151 70.4925) (end 156.985 70.4925) (width 0.2) (layer "F.Cu") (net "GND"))
 (segment (start 169 58.4775) (end 156.985 70.4925) (width 0.2) (layer "F.Cu") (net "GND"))
 (segment (start 167.8 113) (end 183.8 97) (width 0.2) (layer "F.Cu") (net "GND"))
 (segment (start 155.624314 45.75) (end 155.907158 46.032843) (width 0.2) (layer "F.Cu") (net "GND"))
 (segment (start 156.19 52.94) (end 157.25 54) (width 0.2) (layer "F.Cu") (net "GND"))
 (segment (start 151 70.4925) (end 151 86.16) (width 0.2) (layer "F.Cu") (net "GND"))
 (segment (start 169 55) (end 169 58.4775) (width 0.2) (layer "F.Cu") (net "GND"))
 (segment (start 150.54 113) (end 137.35 99.81) (width 0.2) (layer "F.Cu") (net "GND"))
 (segment (start 150 69.54) (end 150.9525 70.4925) (width 0.2) (layer "F.Cu") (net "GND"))
 (segment (start 168 54) (end 169 55) (width 0.2) (layer "F.Cu") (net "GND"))
 (segment (start 152.81 45.75) (end 156.19 45.75) (width 0.2) (layer "F.Cu") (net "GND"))
 (segment (start 156.19 45.75) (end 163.81 45.75) (width 0.2) (layer "F.Cu") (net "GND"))
 (segment (start 150.54 113) (end 167.8 113) (width 0.2) (layer "F.Cu") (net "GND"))
 (segment (start 137.35 99.81) (end 131.5 99.81) (width 0.2) (layer "F.Cu") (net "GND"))
 (segment (start 145.19 58.25) (end 145.19 55.19) (width 0.2) (layer "F.Cu") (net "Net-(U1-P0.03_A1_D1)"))
 (segment (start 145.19 55.19) (end 142 52) (width 0.2) (layer "F.Cu") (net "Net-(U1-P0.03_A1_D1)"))
 (segment (start 124 57) (end 124 64) (width 0.2) (layer "F.Cu") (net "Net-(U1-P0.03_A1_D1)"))
 (segment (start 124 64) (end 130.4925 70.4925) (width 0.2) (layer "F.Cu") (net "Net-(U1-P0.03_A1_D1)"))
 (segment (start 130.4925 70.4925) (end 140.475 70.4925) (width 0.2) (layer "F.Cu") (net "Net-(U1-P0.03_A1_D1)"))
 (segment (start 145.19 58.25) (end 152.81 58.25) (width 0.2) (layer "F.Cu") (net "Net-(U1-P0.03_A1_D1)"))
 (segment (start 142 52) (end 129 52) (width 0.2) (layer "F.Cu") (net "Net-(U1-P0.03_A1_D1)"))
 (segment (start 129 52) (end 124 57) (width 0.2) (layer "F.Cu") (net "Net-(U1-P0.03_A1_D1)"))
 (segment (start 134.107793 45.698655) (end 141.727793 45.698655) (width 0.2) (layer "F.Cu") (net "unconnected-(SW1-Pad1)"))
 (segment (start 134.107793 58.198655) (end 141.727793 58.198655) (width 0.2) (layer "F.Cu") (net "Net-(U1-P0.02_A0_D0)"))
 (segment (start 141.727793 66.699707) (end 140.475 67.9525) (width 0.2) (layer "F.Cu") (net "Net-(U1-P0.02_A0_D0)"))
 (segment (start 141.727793 58.198655) (end 141.727793 66.699707) (width 0.2) (layer "F.Cu") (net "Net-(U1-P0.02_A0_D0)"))
 (segment (start 176.2 93.7715) (end 158.001 75.5725) (width 0.2) (layer "F.Cu") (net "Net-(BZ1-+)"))
 (segment (start 158.001 75.5725) (end 156.985 75.5725) (width 0.2) (layer "F.Cu") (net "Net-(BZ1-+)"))
 (segment (start 176.2 97) (end 176.2 93.7715) (width 0.2) (layer "F.Cu") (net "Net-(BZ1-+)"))
 (segment (start 144 69.5075) (end 140.475 73.0325) (width 0.2) (layer "F.Cu") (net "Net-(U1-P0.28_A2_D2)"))
 (segment (start 144 67) (end 144 69.5075) (width 0.2) (layer "F.Cu") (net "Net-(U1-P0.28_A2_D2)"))
 (segment (start 156 63) (end 148 63) (width 0.2) (layer "F.Cu") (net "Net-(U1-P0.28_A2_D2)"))
 (segment (start 156.19 58.25) (end 156 58.44) (width 0.2) (layer "F.Cu") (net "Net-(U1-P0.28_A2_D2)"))
 (segment (start 156.19 58.25) (end 163.81 58.25) (width 0.2) (layer "F.Cu") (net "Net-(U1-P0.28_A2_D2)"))
 (segment (start 148 63) (end 144 67) (width 0.2) (layer "F.Cu") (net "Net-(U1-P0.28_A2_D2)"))
 (segment (start 156 58.44) (end 156 61) (width 0.2) (layer "F.Cu") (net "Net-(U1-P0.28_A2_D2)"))
 (segment (start 163.244314 58.25) (end 163.527157 57.967157) (width 0.2) (layer "F.Cu") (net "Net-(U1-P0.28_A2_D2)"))
 (via (at 156 63) (size 0.6) (drill 0.3) (layers "F.Cu" "B.Cu") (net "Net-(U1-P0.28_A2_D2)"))
 (via (at 156 61) (size 0.6) (drill 0.3) (layers "F.Cu" "B.Cu") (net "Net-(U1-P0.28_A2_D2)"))
 (segment (start 156 61) (end 156 63) (width 0.2) (layer "B.Cu") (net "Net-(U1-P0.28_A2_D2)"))
 (segment (start 131.5 92.19) (end 131.5 86.0715) (width 0.2) (layer "F.Cu") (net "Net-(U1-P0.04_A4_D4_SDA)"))
 (segment (start 131.5 86.0715) (end 139.459 78.1125) (width 0.2) (layer "F.Cu") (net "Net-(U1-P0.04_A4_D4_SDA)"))
 (segment (start 139.459 78.1125) (end 140.475 78.1125) (width 0.2) (layer "F.Cu") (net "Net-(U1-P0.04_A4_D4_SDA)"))
 (segment (start 139.3475 80.6525) (end 140.475 80.6525) (width 0.2) (layer "F.Cu") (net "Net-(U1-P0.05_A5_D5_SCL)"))
 (segment (start 133 87) (end 139.3475 80.6525) (width 0.2) (layer "F.Cu") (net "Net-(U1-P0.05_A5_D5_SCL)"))
 (segment (start 133 93.23) (end 133 87) (width 0.2) (layer "F.Cu") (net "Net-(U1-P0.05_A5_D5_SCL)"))
 (segment (start 131.5 94.73) (end 133 93.23) (width 0.2) (layer "F.Cu") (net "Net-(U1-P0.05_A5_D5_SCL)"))
 (segment (start 131.5 97.27) (end 144.77 84) (width 0.2) (layer "F.Cu") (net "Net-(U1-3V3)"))
 (segment (start 154 76.0175) (end 154 82) (width 0.2) (layer "F.Cu") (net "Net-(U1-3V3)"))
 (segment (start 154 82) (end 152 84) (width 0.2) (layer "F.Cu") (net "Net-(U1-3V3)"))
 (segment (start 156.985 73.0325) (end 154 76.0175) (width 0.2) (layer "F.Cu") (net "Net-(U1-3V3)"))
 (segment (start 144.77 84) (end 149 84) (width 0.2) (layer "F.Cu") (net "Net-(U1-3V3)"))
 (via (at 149 84) (size 0.6) (drill 0.3) (layers "F.Cu" "B.Cu") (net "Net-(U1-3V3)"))
 (via (at 152 84) (size 0.6) (drill 0.3) (layers "F.Cu" "B.Cu") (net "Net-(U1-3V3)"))
 (segment (start 149 84) (end 152 84) (width 0.2) (layer "B.Cu") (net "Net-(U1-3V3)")))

